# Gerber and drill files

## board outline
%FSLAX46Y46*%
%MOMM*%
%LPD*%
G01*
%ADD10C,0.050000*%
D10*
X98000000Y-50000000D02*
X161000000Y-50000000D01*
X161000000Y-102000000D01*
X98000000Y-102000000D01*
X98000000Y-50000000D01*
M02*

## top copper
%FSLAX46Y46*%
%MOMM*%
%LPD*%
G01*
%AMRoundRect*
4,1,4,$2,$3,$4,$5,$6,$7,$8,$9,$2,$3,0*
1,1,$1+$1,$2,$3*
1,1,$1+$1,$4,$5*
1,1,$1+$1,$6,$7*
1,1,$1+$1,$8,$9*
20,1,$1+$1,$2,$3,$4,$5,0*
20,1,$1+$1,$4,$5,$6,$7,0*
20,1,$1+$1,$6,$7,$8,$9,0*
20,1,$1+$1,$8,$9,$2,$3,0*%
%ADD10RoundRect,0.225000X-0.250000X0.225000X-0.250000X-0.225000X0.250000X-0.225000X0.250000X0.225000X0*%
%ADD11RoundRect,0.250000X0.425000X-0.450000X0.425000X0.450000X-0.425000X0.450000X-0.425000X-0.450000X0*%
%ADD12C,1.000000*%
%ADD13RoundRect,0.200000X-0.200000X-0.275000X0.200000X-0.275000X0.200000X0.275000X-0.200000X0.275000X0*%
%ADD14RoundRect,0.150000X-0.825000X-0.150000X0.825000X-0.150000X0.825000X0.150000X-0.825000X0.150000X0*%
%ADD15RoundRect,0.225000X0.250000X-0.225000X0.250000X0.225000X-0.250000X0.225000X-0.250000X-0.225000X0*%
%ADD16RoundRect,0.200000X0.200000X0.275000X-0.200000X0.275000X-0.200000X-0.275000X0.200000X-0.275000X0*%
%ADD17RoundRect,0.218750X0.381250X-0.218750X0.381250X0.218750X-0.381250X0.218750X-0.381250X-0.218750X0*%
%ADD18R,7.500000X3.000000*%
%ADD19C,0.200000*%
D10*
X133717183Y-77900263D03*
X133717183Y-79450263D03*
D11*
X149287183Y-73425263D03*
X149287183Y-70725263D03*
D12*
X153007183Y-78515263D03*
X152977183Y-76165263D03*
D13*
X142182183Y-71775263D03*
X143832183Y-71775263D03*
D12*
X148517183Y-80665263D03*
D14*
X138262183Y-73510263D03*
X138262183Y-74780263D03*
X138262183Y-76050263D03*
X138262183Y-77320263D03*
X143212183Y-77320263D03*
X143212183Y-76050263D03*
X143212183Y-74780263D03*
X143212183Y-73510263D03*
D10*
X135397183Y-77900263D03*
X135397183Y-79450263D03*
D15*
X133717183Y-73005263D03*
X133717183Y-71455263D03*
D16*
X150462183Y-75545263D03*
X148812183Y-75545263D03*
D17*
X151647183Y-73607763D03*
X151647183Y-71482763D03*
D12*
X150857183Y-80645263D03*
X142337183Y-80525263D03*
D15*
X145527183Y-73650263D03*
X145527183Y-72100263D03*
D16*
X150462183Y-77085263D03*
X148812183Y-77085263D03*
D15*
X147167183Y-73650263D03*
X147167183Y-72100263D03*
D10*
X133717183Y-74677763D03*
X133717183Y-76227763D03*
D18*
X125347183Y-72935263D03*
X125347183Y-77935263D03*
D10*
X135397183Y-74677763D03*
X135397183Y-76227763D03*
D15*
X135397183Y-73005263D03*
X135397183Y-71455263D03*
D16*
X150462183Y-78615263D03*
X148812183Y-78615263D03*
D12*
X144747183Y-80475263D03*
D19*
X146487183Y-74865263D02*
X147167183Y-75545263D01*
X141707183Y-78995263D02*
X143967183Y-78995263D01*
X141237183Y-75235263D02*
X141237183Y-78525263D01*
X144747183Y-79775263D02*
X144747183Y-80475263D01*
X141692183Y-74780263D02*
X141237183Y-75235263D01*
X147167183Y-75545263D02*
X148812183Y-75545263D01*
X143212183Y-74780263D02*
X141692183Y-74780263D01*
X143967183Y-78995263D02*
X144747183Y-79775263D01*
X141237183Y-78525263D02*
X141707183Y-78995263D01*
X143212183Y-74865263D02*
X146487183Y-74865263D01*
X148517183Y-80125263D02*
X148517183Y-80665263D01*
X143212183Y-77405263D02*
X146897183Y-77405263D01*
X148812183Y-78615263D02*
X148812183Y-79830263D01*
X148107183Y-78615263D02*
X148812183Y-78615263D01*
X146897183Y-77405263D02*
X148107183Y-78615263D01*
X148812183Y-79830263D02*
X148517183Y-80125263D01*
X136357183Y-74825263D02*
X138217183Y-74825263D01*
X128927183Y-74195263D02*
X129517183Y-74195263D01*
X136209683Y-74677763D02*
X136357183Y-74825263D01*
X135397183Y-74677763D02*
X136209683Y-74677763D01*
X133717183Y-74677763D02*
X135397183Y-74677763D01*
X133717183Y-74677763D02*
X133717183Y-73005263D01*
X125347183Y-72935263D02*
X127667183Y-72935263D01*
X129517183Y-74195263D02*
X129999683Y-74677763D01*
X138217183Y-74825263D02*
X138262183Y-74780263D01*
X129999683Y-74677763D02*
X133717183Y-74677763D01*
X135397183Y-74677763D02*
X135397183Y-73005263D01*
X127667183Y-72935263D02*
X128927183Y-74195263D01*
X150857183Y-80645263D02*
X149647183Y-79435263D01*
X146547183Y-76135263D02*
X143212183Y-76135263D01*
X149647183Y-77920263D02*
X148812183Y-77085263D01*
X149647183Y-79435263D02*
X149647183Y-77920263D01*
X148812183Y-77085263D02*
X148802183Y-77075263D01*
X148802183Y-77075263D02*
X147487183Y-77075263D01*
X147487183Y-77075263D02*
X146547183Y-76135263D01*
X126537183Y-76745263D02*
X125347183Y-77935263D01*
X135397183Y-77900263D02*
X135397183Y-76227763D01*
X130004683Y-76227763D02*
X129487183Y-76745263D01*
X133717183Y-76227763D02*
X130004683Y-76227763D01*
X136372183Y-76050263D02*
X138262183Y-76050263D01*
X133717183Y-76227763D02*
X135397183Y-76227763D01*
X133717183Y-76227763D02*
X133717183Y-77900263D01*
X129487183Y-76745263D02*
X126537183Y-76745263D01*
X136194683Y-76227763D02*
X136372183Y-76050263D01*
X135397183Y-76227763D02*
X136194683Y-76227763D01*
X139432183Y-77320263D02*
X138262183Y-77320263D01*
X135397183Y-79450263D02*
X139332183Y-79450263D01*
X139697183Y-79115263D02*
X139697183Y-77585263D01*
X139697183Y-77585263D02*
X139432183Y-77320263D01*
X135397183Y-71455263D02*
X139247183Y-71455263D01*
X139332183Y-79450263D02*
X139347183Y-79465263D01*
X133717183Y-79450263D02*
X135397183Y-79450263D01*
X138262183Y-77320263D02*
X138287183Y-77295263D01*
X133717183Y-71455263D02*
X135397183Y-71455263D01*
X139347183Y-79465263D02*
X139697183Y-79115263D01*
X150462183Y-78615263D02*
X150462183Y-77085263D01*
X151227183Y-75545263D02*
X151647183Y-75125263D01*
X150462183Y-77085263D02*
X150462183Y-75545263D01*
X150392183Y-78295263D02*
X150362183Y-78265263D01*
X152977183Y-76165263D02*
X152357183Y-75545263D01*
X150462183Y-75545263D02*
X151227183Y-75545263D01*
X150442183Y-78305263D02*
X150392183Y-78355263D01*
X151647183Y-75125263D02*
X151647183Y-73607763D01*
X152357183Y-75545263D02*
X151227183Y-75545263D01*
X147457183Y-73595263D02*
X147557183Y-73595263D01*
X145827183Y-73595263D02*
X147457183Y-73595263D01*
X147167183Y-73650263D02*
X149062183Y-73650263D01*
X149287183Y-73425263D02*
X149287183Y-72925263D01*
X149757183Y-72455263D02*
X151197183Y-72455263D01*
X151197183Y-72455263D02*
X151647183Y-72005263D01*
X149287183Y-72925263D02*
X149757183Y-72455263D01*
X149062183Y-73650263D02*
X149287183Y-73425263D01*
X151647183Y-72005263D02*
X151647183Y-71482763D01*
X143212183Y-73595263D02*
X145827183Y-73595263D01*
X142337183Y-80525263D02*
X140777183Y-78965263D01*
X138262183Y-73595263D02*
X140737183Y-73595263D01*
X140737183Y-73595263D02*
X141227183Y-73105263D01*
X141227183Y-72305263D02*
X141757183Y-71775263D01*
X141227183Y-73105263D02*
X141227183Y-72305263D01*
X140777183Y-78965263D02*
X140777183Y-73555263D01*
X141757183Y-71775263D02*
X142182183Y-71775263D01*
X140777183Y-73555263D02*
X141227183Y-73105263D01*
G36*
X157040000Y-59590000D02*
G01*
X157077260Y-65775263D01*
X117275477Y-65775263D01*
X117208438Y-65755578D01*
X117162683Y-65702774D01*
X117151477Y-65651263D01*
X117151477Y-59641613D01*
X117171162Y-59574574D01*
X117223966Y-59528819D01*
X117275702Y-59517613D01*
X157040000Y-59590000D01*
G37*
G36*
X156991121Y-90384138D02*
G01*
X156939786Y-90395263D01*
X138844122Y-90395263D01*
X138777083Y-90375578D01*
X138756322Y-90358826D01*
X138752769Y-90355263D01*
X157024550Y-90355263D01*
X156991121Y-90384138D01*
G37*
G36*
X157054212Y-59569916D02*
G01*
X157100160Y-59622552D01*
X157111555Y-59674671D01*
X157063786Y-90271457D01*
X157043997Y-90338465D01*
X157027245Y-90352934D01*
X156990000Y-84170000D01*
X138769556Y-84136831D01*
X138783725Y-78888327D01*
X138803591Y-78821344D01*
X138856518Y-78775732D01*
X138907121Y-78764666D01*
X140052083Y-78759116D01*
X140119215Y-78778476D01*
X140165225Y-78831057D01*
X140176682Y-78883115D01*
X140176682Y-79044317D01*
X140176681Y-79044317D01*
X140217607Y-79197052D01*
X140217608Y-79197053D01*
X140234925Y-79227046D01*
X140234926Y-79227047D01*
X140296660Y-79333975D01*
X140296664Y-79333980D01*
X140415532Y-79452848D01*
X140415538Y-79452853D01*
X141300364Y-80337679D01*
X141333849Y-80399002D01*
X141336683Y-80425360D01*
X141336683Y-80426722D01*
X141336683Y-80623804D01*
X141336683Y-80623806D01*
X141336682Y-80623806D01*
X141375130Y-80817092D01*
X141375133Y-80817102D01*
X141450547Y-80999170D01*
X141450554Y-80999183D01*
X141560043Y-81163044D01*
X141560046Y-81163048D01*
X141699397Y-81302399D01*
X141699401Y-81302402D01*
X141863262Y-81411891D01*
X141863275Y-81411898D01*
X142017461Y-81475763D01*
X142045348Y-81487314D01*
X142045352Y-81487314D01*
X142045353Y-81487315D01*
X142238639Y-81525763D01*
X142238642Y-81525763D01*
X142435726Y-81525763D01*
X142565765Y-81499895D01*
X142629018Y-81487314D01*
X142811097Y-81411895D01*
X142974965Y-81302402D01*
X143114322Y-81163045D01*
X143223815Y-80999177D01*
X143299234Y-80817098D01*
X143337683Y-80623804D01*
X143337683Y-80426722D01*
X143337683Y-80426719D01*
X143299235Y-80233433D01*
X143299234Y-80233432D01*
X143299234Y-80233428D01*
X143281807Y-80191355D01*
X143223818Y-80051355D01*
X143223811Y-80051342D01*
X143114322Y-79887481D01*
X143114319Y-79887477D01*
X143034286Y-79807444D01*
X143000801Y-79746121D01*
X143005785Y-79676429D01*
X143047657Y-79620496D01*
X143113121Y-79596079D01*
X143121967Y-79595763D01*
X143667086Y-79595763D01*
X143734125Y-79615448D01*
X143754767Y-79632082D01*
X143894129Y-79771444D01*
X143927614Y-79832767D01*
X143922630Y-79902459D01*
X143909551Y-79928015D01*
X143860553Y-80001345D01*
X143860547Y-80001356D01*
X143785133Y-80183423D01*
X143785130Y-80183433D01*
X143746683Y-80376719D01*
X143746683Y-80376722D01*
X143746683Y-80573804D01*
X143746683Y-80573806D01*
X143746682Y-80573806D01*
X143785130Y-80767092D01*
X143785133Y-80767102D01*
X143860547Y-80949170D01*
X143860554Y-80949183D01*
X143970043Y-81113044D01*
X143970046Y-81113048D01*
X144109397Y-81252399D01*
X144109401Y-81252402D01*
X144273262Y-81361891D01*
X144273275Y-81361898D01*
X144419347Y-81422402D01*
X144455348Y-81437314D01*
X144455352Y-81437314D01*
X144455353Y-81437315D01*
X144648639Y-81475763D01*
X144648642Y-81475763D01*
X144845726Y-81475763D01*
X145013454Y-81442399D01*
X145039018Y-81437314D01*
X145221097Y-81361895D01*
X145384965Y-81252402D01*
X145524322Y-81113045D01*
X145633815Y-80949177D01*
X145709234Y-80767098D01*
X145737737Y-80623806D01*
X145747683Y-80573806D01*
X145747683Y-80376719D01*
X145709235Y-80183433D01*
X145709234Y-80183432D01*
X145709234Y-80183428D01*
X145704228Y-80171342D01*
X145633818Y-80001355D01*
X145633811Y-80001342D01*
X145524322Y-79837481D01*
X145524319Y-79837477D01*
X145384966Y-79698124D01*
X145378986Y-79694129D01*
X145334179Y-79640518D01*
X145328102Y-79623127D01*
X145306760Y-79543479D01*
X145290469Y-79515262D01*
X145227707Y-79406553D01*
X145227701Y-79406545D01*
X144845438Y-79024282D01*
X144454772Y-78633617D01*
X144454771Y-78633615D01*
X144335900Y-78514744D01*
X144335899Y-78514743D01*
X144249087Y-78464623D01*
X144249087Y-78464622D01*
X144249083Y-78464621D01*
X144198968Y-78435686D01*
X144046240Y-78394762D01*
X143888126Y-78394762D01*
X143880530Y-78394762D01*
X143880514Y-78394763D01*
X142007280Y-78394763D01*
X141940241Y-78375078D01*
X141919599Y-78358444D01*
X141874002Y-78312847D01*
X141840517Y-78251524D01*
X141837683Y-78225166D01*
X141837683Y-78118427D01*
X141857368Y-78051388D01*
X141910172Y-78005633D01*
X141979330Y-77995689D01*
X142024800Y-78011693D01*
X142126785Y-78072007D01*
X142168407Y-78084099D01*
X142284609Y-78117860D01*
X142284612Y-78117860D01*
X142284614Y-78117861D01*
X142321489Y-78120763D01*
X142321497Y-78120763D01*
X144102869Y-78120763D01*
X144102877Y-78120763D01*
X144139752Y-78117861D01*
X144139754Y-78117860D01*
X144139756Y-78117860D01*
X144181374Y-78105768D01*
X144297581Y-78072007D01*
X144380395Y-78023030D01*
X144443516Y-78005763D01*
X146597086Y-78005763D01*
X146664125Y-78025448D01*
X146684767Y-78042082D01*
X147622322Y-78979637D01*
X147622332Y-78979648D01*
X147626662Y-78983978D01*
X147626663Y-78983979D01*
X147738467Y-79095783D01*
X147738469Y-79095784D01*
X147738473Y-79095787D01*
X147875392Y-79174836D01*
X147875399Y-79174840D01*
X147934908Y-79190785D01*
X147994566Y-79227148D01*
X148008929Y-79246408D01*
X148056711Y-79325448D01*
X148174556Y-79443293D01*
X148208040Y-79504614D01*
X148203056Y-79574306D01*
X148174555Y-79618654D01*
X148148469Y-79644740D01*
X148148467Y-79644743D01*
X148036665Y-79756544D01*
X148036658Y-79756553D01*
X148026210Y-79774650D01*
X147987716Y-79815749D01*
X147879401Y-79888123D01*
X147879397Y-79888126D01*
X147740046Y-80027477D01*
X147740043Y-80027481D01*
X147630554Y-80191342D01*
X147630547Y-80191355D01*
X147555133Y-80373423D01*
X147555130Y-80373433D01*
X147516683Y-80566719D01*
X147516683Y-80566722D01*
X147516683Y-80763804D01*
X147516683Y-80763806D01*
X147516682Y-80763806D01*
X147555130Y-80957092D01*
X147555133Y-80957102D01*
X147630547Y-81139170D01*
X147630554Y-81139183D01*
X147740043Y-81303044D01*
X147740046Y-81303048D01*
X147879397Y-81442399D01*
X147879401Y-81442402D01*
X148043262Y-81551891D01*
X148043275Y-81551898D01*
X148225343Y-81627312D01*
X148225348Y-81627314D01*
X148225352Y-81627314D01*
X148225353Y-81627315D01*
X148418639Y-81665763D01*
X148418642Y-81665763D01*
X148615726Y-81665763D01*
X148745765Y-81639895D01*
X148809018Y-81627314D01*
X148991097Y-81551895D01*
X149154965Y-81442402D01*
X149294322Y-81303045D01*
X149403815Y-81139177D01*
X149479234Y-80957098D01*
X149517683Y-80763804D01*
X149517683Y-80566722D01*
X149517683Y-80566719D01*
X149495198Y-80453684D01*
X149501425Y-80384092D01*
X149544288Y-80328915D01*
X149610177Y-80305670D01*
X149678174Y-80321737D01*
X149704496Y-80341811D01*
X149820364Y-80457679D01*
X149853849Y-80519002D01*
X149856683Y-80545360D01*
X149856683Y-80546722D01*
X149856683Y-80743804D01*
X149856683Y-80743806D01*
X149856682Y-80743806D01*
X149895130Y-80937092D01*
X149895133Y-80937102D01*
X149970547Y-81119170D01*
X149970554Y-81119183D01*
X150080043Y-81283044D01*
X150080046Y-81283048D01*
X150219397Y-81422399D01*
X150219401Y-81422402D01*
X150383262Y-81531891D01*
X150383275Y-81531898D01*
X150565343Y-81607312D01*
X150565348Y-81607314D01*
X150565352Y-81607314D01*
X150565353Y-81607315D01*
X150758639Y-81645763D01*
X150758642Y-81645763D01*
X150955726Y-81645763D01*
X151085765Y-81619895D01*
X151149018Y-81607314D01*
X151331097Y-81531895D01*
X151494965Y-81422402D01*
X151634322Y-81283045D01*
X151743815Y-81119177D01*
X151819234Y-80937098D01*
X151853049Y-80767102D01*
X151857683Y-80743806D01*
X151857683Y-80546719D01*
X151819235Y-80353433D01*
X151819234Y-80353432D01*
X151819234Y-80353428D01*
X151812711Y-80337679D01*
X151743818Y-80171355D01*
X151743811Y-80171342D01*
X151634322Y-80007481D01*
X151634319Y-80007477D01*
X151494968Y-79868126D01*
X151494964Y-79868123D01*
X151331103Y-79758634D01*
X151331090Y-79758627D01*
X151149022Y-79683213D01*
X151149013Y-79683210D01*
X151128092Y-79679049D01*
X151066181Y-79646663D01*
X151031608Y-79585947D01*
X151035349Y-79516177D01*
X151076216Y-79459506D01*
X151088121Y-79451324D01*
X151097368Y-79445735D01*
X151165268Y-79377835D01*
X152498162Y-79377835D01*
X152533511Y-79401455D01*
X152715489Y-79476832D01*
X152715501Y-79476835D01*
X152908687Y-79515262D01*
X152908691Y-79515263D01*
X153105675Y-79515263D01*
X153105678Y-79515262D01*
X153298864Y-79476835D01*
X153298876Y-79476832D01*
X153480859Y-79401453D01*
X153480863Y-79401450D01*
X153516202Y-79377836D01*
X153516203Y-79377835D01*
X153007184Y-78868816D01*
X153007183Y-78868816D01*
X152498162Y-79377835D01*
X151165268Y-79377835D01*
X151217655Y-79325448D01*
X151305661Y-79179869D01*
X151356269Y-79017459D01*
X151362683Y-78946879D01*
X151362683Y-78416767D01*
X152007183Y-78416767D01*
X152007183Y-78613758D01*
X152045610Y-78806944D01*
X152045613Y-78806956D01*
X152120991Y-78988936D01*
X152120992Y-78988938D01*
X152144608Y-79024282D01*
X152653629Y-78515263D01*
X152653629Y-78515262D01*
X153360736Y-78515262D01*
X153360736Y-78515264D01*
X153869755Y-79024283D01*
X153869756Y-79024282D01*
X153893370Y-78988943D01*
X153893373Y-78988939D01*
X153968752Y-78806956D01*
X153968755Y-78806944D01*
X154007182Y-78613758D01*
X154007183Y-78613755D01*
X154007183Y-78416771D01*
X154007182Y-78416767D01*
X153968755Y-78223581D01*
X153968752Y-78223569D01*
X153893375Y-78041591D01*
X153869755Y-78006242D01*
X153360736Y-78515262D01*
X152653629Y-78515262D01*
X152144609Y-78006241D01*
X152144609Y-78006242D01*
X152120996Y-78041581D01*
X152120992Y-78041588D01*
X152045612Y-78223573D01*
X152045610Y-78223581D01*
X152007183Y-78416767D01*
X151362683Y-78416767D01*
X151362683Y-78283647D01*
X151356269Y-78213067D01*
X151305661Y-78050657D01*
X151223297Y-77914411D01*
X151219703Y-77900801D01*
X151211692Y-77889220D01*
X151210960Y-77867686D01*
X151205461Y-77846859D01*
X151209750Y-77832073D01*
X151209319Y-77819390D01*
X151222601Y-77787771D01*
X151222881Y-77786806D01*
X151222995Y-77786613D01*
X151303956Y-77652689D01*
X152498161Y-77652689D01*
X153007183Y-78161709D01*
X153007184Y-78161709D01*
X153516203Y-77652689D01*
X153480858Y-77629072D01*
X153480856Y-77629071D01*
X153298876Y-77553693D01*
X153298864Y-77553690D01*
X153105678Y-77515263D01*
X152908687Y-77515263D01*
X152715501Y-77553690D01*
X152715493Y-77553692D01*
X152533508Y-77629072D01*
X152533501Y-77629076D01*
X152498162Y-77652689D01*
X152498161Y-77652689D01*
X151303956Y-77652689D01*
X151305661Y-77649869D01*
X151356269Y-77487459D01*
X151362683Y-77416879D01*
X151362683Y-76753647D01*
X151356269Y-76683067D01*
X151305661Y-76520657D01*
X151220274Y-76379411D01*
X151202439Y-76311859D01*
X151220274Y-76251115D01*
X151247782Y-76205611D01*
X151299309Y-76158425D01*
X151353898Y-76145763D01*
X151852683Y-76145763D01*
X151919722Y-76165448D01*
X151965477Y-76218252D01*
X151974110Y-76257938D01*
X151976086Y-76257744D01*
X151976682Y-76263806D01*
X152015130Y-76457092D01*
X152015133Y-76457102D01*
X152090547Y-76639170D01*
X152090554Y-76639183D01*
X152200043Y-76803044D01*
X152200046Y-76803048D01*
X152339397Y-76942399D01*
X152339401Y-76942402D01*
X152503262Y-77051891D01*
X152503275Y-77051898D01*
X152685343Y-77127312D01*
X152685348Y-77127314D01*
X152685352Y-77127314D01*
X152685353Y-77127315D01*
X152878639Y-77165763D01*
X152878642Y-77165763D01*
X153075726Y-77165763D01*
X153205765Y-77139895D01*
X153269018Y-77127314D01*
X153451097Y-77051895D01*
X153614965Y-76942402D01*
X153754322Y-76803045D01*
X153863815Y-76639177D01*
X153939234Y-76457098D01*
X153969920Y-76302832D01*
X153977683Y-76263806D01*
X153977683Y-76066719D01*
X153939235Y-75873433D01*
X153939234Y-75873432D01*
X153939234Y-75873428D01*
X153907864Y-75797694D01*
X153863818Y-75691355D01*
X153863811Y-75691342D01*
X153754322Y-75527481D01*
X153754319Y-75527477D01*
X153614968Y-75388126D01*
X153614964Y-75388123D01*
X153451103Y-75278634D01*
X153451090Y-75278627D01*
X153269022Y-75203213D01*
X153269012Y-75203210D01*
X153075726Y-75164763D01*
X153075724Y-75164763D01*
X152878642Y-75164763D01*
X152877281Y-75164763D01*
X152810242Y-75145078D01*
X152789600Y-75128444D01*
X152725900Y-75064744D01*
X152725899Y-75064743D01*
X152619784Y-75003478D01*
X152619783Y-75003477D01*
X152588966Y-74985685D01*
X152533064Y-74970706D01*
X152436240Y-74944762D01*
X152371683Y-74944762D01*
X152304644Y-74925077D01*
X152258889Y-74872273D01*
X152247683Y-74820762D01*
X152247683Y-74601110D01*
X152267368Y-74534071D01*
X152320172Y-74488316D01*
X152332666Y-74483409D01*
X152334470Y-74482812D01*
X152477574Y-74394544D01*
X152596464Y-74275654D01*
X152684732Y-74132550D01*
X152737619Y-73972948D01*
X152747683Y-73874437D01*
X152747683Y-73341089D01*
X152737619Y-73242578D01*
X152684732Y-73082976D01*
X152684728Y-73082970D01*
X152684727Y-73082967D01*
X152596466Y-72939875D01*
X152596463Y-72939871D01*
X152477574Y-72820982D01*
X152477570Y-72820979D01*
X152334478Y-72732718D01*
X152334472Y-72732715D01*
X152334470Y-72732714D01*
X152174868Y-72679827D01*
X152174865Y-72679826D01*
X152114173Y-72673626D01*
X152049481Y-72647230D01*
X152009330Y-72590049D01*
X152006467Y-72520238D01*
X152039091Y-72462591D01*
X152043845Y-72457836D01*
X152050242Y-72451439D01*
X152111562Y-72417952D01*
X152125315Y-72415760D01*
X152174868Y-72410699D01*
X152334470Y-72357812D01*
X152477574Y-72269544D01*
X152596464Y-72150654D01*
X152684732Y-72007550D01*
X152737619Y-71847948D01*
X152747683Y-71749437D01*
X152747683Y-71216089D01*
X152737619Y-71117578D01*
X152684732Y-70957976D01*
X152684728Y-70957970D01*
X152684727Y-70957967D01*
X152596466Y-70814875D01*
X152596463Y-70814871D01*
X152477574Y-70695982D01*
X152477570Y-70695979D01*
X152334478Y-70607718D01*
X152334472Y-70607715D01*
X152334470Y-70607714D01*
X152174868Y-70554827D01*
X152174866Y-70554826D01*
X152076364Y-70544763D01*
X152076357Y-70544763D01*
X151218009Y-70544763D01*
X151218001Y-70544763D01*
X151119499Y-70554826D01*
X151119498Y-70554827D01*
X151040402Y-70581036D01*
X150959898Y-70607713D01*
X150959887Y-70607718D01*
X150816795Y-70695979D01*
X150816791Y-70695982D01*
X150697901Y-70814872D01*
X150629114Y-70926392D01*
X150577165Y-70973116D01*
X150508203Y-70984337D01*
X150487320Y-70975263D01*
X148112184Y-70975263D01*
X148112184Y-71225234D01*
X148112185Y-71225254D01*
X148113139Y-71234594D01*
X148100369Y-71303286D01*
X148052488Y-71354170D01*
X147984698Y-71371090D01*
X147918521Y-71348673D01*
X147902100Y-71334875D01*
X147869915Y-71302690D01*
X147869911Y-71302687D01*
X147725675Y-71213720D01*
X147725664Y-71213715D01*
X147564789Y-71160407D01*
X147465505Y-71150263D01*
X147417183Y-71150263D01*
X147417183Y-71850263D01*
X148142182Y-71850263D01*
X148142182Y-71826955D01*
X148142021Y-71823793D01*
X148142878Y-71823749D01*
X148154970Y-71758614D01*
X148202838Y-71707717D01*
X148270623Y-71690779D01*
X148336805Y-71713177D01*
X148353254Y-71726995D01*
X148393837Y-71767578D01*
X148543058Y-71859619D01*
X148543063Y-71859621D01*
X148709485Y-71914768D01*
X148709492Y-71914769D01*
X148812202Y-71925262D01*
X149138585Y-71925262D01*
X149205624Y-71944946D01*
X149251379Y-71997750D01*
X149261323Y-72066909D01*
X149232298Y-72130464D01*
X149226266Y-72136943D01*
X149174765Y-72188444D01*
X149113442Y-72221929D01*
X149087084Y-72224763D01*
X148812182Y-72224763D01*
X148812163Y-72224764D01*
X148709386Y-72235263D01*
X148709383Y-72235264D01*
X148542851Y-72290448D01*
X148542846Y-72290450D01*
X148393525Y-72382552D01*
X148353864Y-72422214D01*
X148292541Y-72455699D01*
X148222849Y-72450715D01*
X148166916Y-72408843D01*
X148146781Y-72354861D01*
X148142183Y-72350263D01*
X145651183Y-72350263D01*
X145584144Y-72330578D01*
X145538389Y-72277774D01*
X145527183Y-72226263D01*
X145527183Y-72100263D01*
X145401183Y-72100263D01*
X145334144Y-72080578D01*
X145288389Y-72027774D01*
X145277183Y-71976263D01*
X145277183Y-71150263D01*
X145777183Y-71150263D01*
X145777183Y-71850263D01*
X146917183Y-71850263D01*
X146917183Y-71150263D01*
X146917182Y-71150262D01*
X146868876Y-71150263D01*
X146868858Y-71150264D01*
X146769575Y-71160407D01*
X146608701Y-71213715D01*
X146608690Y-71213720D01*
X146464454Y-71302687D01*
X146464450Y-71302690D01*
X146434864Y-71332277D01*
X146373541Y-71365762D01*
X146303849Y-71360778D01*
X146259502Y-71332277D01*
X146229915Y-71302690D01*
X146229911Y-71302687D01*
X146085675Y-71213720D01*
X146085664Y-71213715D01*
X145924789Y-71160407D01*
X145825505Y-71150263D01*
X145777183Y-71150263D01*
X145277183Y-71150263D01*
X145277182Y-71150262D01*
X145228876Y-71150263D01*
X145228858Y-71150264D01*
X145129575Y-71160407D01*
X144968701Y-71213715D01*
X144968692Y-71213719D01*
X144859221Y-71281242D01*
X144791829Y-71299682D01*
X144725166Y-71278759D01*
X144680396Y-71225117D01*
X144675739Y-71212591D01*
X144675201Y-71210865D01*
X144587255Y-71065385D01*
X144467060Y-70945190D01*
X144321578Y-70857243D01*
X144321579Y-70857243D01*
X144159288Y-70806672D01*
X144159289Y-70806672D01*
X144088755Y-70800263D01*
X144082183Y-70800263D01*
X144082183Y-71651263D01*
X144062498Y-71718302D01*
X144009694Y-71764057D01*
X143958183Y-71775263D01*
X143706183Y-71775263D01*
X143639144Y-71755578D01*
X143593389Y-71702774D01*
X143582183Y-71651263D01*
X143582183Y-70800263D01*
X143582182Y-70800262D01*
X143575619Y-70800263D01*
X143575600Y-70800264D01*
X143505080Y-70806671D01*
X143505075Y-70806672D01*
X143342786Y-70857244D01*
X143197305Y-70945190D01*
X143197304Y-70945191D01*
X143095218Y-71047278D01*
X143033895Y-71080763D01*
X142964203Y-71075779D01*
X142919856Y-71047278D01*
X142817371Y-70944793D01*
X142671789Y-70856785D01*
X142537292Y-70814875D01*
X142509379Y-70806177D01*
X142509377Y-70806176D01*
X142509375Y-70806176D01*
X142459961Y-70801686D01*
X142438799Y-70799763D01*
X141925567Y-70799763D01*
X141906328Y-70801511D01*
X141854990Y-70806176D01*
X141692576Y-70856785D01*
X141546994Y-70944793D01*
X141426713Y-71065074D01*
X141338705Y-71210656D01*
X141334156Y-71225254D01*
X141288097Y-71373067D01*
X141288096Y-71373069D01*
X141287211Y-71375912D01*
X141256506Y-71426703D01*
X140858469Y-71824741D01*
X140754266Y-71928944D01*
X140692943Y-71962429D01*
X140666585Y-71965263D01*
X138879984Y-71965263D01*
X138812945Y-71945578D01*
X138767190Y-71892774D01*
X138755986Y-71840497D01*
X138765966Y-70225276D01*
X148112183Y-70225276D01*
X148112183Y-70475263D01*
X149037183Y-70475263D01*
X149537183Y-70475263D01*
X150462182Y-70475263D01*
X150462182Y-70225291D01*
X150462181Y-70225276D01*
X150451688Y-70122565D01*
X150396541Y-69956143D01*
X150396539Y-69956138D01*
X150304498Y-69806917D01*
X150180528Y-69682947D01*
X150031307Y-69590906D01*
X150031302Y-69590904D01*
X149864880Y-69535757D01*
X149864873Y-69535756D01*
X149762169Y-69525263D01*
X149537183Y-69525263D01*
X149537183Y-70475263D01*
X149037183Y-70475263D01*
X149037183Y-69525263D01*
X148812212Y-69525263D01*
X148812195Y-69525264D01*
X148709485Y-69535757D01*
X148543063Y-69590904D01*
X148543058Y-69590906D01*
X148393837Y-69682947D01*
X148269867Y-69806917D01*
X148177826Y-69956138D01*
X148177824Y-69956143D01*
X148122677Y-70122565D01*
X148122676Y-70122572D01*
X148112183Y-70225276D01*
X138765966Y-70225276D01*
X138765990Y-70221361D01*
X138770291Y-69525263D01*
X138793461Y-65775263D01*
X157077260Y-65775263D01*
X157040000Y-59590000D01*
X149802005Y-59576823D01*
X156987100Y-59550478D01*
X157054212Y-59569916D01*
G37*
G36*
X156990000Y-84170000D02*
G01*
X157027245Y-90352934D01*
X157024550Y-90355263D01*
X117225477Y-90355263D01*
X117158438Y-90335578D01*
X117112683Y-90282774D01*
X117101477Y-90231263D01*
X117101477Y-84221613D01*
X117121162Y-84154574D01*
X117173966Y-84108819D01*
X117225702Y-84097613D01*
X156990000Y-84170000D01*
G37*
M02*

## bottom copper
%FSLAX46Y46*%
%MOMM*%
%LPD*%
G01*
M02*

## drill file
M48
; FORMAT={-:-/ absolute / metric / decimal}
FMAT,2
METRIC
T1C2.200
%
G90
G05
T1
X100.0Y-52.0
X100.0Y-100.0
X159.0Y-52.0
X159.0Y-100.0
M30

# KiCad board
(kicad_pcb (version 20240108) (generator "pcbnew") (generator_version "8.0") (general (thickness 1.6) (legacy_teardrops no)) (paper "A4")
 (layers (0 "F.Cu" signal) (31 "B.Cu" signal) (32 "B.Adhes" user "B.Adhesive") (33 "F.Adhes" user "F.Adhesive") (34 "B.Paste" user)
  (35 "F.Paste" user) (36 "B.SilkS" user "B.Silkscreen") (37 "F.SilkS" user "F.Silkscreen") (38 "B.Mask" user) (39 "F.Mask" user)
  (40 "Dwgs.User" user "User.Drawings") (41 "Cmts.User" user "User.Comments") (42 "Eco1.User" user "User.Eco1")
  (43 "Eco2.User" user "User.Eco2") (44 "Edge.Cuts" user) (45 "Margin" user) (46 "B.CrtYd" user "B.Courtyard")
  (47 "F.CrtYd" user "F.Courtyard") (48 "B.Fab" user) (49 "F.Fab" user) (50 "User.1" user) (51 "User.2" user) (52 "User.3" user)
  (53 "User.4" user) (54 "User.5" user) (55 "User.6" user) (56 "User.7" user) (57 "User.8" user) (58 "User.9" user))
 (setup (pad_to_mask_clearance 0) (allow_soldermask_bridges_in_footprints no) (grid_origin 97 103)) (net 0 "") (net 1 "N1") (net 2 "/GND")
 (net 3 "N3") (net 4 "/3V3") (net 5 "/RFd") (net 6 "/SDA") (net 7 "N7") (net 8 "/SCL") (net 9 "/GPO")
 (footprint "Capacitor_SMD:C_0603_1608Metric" (layer "F.Cu") (at 133.717183 78.675263 -90)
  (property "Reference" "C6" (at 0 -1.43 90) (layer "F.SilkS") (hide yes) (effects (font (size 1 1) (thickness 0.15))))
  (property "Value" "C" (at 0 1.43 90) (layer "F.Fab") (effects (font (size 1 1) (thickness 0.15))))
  (pad "1" smd roundrect (at -0.775 0 270) (size 0.9 0.95) (layers "F.Cu" "F.Paste" "F.Mask") (roundrect_rratio 0.25) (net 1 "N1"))
  (pad "2" smd roundrect (at 0.775 0 270) (size 0.9 0.95) (layers "F.Cu" "F.Paste" "F.Mask") (roundrect_rratio 0.25) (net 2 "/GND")))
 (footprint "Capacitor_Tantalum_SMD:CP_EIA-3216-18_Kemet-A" (layer "F.Cu") (at 149.287183 72.075263 90)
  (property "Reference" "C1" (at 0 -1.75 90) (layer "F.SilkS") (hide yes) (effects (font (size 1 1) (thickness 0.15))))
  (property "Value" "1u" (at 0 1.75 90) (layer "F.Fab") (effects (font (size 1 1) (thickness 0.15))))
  (pad "1" smd roundrect (at -1.35 0 90) (size 1.4 1.35) (layers "F.Cu" "F.Paste" "F.Mask") (roundrect_rratio 0.185185) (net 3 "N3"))
  (pad "2" smd roundrect (at 1.35 0 90) (size 1.4 1.35) (layers "F.Cu" "F.Paste" "F.Mask") (roundrect_rratio 0.185185) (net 2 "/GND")))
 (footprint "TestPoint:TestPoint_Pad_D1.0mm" (layer "F.Cu") (at 153.007183 78.515263)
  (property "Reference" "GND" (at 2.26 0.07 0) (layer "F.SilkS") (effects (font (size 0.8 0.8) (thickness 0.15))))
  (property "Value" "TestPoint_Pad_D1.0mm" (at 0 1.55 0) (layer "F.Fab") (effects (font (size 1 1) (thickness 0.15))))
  (pad "1" smd circle (at 0 0) (size 1 1) (layers "F.Cu" "F.Mask") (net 2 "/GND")))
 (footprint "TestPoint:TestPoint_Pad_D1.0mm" (layer "F.Cu") (at 152.977183 76.165263)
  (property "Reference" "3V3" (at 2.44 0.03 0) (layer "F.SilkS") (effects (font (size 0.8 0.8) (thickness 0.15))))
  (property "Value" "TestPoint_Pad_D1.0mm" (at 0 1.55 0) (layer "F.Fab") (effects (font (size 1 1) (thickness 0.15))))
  (pad "2" smd circle (at 0 0) (size 1 1) (layers "F.Cu" "F.Mask") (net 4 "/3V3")))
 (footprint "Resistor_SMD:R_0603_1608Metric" (layer "F.Cu") (at 143.007183 71.775263)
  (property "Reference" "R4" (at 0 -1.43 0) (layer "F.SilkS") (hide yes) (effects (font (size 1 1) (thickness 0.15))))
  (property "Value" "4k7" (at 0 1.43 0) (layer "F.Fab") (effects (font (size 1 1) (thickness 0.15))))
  (pad "1" smd roundrect (at -0.825 0) (size 0.8 0.95) (layers "F.Cu" "F.Paste" "F.Mask") (roundrect_rratio 0.25) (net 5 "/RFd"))
  (pad "2" smd roundrect (at 0.825 0) (size 0.8 0.95) (layers "F.Cu" "F.Paste" "F.Mask") (roundrect_rratio 0.25) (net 2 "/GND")))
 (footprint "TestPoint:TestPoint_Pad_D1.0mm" (layer "F.Cu") (at 148.517183 80.665263)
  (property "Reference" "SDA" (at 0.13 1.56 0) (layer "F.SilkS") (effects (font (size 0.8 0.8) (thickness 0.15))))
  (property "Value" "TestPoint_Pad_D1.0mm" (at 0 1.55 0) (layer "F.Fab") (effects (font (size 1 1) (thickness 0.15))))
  (pad "3" smd circle (at 0 0) (size 1 1) (layers "F.Cu" "F.Mask") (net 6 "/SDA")))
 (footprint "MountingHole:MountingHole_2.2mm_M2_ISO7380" (layer "F.Cu") (at 100 52)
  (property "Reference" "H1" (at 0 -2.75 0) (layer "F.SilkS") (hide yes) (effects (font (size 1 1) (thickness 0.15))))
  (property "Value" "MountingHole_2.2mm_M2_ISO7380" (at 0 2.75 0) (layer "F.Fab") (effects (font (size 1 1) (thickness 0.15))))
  (pad "" np_thru_hole circle (at 0 0) (size 2.2 2.2) (drill 2.2) (layers "*.Cu" "*.Mask")))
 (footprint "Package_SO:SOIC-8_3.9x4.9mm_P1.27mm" (layer "F.Cu") (at 140.737183 75.415263)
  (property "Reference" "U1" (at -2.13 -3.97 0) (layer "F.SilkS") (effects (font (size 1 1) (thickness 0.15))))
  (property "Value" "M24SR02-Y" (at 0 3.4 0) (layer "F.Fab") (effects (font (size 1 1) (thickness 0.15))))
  (pad "1" smd roundrect (at -2.475 -1.905) (size 1.95 0.6) (layers "F.Cu" "F.Paste" "F.Mask") (roundrect_rratio 0.25) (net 5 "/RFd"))
  (pad "2" smd roundrect (at -2.475 -0.635) (size 1.95 0.6) (layers "F.Cu" "F.Paste" "F.Mask") (roundrect_rratio 0.25) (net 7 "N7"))
  (pad "3" smd roundrect (at -2.475 0.635) (size 1.95 0.6) (layers "F.Cu" "F.Paste" "F.Mask") (roundrect_rratio 0.25) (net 1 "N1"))
  (pad "4" smd roundrect (at -2.475 1.905) (size 1.95 0.6) (layers "F.Cu" "F.Paste" "F.Mask") (roundrect_rratio 0.25) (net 2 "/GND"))
  (pad "5" smd roundrect (at 2.475 1.905) (size 1.95 0.6) (layers "F.Cu" "F.Paste" "F.Mask") (roundrect_rratio 0.25) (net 6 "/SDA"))
  (pad "6" smd roundrect (at 2.475 0.635) (size 1.95 0.6) (layers "F.Cu" "F.Paste" "F.Mask") (roundrect_rratio 0.25) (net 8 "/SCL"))
  (pad "7" smd roundrect (at 2.475 -0.635) (size 1.95 0.6) (layers "F.Cu" "F.Paste" "F.Mask") (roundrect_rratio 0.25) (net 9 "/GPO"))
  (pad "8" smd roundrect (at 2.475 -1.905) (size 1.95 0.6) (layers "F.Cu" "F.Paste" "F.Mask") (roundrect_rratio 0.25) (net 3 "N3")))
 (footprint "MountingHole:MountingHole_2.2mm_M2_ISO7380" (layer "F.Cu") (at 159 100)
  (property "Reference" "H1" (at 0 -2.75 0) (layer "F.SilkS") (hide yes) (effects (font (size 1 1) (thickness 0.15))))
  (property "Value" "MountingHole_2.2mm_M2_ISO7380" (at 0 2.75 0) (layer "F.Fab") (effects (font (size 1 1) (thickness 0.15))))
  (pad "" np_thru_hole circle (at 0 0) (size 2.2 2.2) (drill 2.2) (layers "*.Cu" "*.Mask")))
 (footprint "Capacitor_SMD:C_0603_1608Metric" (layer "F.Cu") (at 135.397183 78.675263 -90)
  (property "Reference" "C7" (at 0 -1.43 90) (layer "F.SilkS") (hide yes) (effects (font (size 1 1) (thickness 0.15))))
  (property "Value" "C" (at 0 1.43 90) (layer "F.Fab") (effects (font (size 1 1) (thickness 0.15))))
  (pad "1" smd roundrect (at -0.775 0 270) (size 0.9 0.95) (layers "F.Cu" "F.Paste" "F.Mask") (roundrect_rratio 0.25) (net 1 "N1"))
  (pad "2" smd roundrect (at 0.775 0 270) (size 0.9 0.95) (layers "F.Cu" "F.Paste" "F.Mask") (roundrect_rratio 0.25) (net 2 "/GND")))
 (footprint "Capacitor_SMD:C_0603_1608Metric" (layer "F.Cu") (at 133.717183 72.230263 90)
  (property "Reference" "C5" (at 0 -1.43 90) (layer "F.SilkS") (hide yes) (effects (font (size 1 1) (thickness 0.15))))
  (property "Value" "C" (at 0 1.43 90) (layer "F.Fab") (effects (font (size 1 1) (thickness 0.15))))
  (pad "1" smd roundrect (at -0.775 0 90) (size 0.9 0.95) (layers "F.Cu" "F.Paste" "F.Mask") (roundrect_rratio 0.25) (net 7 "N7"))
  (pad "2" smd roundrect (at 0.775 0 90) (size 0.9 0.95) (layers "F.Cu" "F.Paste" "F.Mask") (roundrect_rratio 0.25) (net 2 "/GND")))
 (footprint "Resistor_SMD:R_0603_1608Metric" (layer "F.Cu") (at 149.637183 75.545263 180)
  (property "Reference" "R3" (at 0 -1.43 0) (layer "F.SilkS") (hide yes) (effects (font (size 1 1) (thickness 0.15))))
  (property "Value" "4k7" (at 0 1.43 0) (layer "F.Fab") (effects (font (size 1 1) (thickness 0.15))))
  (pad "1" smd roundrect (at -0.825 0 180) (size 0.8 0.95) (layers "F.Cu" "F.Paste" "F.Mask") (roundrect_rratio 0.25) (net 4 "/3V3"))
  (pad "2" smd roundrect (at 0.825 0 180) (size 0.8 0.95) (layers "F.Cu" "F.Paste" "F.Mask") (roundrect_rratio 0.25) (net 9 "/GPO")))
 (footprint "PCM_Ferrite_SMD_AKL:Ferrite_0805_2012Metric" (layer "F.Cu") (at 151.647183 72.545263 90)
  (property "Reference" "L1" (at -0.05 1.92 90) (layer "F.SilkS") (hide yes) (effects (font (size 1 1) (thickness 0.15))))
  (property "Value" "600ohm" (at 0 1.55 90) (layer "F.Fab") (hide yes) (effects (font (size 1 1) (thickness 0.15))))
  (pad "1" smd roundrect (at -1.0625 0 90) (size 0.875 1.2) (layers "F.Cu" "F.Paste" "F.Mask") (roundrect_rratio 0.25) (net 4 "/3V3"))
  (pad "2" smd roundrect (at 1.0625 0 90) (size 0.875 1.2) (layers "F.Cu" "F.Paste" "F.Mask") (roundrect_rratio 0.25) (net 3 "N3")))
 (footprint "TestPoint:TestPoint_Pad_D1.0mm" (layer "F.Cu") (at 150.857183 80.645263)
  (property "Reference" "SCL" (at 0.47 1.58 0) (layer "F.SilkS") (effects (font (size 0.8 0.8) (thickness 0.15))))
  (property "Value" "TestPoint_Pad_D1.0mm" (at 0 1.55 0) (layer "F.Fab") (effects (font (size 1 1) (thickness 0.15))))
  (pad "4" smd circle (at 0 0) (size 1 1) (layers "F.Cu" "F.Mask") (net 8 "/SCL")))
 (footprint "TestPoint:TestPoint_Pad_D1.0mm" (layer "F.Cu") (at 142.337183 80.525263)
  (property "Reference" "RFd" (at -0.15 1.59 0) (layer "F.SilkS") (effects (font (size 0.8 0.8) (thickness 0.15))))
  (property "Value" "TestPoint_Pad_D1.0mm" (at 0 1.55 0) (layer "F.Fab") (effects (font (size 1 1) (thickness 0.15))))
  (pad "6" smd circle (at 0 0) (size 1 1) (layers "F.Cu" "F.Mask") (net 5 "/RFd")))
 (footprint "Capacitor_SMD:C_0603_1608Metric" (layer "F.Cu") (at 145.527183 72.875263 90)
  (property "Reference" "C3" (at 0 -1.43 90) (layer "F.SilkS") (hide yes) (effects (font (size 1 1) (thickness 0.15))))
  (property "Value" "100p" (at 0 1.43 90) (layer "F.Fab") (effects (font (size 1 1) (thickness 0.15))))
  (pad "1" smd roundrect (at -0.775 0 90) (size 0.9 0.95) (layers "F.Cu" "F.Paste" "F.Mask") (roundrect_rratio 0.25) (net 3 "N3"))
  (pad "2" smd roundrect (at 0.775 0 90) (size 0.9 0.95) (layers "F.Cu" "F.Paste" "F.Mask") (roundrect_rratio 0.25) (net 2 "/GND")))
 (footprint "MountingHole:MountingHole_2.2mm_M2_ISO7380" (layer "F.Cu") (at 100 100)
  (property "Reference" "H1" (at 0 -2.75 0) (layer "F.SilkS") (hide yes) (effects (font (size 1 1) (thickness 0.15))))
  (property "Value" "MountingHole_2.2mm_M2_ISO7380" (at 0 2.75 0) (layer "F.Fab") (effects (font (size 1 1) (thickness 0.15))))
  (pad "" np_thru_hole circle (at 0 0) (size 2.2 2.2) (drill 2.2) (layers "*.Cu" "*.Mask")))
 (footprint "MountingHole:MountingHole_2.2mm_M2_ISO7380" (layer "F.Cu") (at 159 52)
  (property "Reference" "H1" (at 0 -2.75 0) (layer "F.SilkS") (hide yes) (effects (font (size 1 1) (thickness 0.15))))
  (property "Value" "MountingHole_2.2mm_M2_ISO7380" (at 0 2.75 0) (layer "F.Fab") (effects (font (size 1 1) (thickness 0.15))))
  (pad "" np_thru_hole circle (at 0 0) (size 2.2 2.2) (drill 2.2) (layers "*.Cu" "*.Mask")))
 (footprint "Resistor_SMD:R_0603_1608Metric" (layer "F.Cu") (at 149.637183 77.085263 180)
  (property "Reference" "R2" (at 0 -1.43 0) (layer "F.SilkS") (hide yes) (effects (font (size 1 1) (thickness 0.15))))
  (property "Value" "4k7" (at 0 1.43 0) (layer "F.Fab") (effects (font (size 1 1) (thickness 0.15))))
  (pad "1" smd roundrect (at -0.825 0 180) (size 0.8 0.95) (layers "F.Cu" "F.Paste" "F.Mask") (roundrect_rratio 0.25) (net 4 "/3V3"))
  (pad "2" smd roundrect (at 0.825 0 180) (size 0.8 0.95) (layers "F.Cu" "F.Paste" "F.Mask") (roundrect_rratio 0.25) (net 8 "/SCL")))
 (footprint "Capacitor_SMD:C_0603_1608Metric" (layer "F.Cu") (at 147.167183 72.875263 90)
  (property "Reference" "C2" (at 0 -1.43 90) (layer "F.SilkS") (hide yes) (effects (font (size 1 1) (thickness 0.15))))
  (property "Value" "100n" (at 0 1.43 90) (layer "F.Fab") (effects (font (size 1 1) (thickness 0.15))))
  (pad "1" smd roundrect (at -0.775 0 90) (size 0.9 0.95) (layers "F.Cu" "F.Paste" "F.Mask") (roundrect_rratio 0.25) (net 3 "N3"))
  (pad "2" smd roundrect (at 0.775 0 90) (size 0.9 0.95) (layers "F.Cu" "F.Paste" "F.Mask") (roundrect_rratio 0.25) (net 2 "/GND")))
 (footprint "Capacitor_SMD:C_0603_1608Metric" (layer "F.Cu") (at 133.717183 75.452763 -90)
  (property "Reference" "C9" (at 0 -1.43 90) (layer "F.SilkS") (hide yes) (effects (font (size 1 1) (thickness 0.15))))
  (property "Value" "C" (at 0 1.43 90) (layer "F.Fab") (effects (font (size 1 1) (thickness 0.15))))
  (pad "1" smd roundrect (at -0.775 0 270) (size 0.9 0.95) (layers "F.Cu" "F.Paste" "F.Mask") (roundrect_rratio 0.25) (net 7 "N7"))
  (pad "2" smd roundrect (at 0.775 0 270) (size 0.9 0.95) (layers "F.Cu" "F.Paste" "F.Mask") (roundrect_rratio 0.25) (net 1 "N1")))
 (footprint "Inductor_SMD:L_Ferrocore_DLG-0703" (layer "F.Cu") (at 125.347183 75.435263 -90)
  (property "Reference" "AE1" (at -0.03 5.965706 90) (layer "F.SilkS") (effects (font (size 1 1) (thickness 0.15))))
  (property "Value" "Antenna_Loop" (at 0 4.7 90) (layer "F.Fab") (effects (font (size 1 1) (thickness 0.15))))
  (pad "1" smd rect (at -2.5 0 270) (size 3 7.5) (layers "F.Cu" "F.Paste" "F.Mask") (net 7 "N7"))
  (pad "2" smd rect (at 2.5 0 270) (size 3 7.5) (layers "F.Cu" "F.Paste" "F.Mask") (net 1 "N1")))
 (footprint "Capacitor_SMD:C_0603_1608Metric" (layer "F.Cu") (at 135.397183 75.452763 -90)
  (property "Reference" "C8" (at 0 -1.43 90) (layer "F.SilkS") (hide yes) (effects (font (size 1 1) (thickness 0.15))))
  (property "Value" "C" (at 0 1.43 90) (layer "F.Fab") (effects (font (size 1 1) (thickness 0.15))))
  (pad "1" smd roundrect (at -0.775 0 270) (size 0.9 0.95) (layers "F.Cu" "F.Paste" "F.Mask") (roundrect_rratio 0.25) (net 7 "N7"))
  (pad "2" smd roundrect (at 0.775 0 270) (size 0.9 0.95) (layers "F.Cu" "F.Paste" "F.Mask") (roundrect_rratio 0.25) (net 1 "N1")))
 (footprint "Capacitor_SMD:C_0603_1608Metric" (layer "F.Cu") (at 135.397183 72.230263 90)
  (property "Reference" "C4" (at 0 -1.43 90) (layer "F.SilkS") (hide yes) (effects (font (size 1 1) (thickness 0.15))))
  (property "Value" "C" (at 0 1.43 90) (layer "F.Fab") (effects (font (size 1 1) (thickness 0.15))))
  (pad "1" smd roundrect (at -0.775 0 90) (size 0.9 0.95) (layers "F.Cu" "F.Paste" "F.Mask") (roundrect_rratio 0.25) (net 7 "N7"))
  (pad "2" smd roundrect (at 0.775 0 90) (size 0.9 0.95) (layers "F.Cu" "F.Paste" "F.Mask") (roundrect_rratio 0.25) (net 2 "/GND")))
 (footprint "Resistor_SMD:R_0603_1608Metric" (layer "F.Cu") (at 149.637183 78.615263 180)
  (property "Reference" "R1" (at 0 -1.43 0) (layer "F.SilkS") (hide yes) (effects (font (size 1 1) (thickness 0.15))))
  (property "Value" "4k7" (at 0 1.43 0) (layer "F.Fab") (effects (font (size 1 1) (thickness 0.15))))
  (pad "1" smd roundrect (at -0.825 0 180) (size 0.8 0.95) (layers "F.Cu" "F.Paste" "F.Mask") (roundrect_rratio 0.25) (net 4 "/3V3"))
  (pad "2" smd roundrect (at 0.825 0 180) (size 0.8 0.95) (layers "F.Cu" "F.Paste" "F.Mask") (roundrect_rratio 0.25) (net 6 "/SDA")))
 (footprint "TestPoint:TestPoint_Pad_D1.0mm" (layer "F.Cu") (at 144.747183 80.475263)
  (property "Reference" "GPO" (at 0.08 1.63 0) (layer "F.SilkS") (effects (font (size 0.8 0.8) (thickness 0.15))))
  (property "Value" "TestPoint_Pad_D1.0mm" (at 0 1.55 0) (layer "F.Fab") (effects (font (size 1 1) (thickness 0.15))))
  (pad "5" smd circle (at 0 0) (size 1 1) (layers "F.Cu" "F.Mask") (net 9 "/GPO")))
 (gr_rect (start 98 50) (end 161 102) (stroke (width 0.05) (type default)) (fill none) (layer "Edge.Cuts"))
 (segment (start 146.487183 74.865263) (end 147.167183 75.545263) (width 0.2) (layer "F.Cu") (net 9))
 (segment (start 141.707183 78.995263) (end 143.967183 78.995263) (width 0.2) (layer "F.Cu") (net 9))
 (segment (start 141.237183 75.235263) (end 141.237183 78.525263) (width 0.2) (layer "F.Cu") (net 9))
 (segment (start 144.747183 79.775263) (end 144.747183 80.475263) (width 0.2) (layer "F.Cu") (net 9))
 (segment (start 141.692183 74.780263) (end 141.237183 75.235263) (width 0.2) (layer "F.Cu") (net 9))
 (segment (start 147.167183 75.545263) (end 148.812183 75.545263) (width 0.2) (layer "F.Cu") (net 9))
 (segment (start 143.212183 74.780263) (end 141.692183 74.780263) (width 0.2) (layer "F.Cu") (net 9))
 (segment (start 143.967183 78.995263) (end 144.747183 79.775263) (width 0.2) (layer "F.Cu") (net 9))
 (segment (start 141.237183 78.525263) (end 141.707183 78.995263) (width 0.2) (layer "F.Cu") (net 9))
 (segment (start 143.212183 74.865263) (end 146.487183 74.865263) (width 0.2) (layer "F.Cu") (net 9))
 (segment (start 148.517183 80.125263) (end 148.517183 80.665263) (width 0.2) (layer "F.Cu") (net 6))
 (segment (start 143.212183 77.405263) (end 146.897183 77.405263) (width 0.2) (layer "F.Cu") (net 6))
 (segment (start 148.812183 78.615263) (end 148.812183 79.830263) (width 0.2) (layer "F.Cu") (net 6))
 (segment (start 148.107183 78.615263) (end 148.812183 78.615263) (width 0.2) (layer "F.Cu") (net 6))
 (segment (start 146.897183 77.405263) (end 148.107183 78.615263) (width 0.2) (layer "F.Cu") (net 6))
 (segment (start 148.812183 79.830263) (end 148.517183 80.125263) (width 0.2) (layer "F.Cu") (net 6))
 (segment (start 136.357183 74.825263) (end 138.217183 74.825263) (width 0.2) (layer "F.Cu") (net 7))
 (segment (start 128.927183 74.195263) (end 129.517183 74.195263) (width 0.2) (layer "F.Cu") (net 7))
 (segment (start 136.209683 74.677763) (end 136.357183 74.825263) (width 0.2) (layer "F.Cu") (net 7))
 (segment (start 135.397183 74.677763) (end 136.209683 74.677763) (width 0.2) (layer "F.Cu") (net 7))
 (segment (start 133.717183 74.677763) (end 135.397183 74.677763) (width 0.2) (layer "F.Cu") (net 7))
 (segment (start 133.717183 74.677763) (end 133.717183 73.005263) (width 0.2) (layer "F.Cu") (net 7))
 (segment (start 125.347183 72.935263) (end 127.667183 72.935263) (width 0.2) (layer "F.Cu") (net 7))
 (segment (start 129.517183 74.195263) (end 129.999683 74.677763) (width 0.2) (layer "F.Cu") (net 7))
 (segment (start 138.217183 74.825263) (end 138.262183 74.780263) (width 0.2) (layer "F.Cu") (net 7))
 (segment (start 129.999683 74.677763) (end 133.717183 74.677763) (width 0.2) (layer "F.Cu") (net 7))
 (segment (start 135.397183 74.677763) (end 135.397183 73.005263) (width 0.2) (layer "F.Cu") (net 7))
 (segment (start 127.667183 72.935263) (end 128.927183 74.195263) (width 0.2) (layer "F.Cu") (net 7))
 (segment (start 150.857183 80.645263) (end 149.647183 79.435263) (width 0.2) (layer "F.Cu") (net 8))
 (segment (start 146.547183 76.135263) (end 143.212183 76.135263) (width 0.2) (layer "F.Cu") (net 8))
 (segment (start 149.647183 77.920263) (end 148.812183 77.085263) (width 0.2) (layer "F.Cu") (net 8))
 (segment (start 149.647183 79.435263) (end 149.647183 77.920263) (width 0.2) (layer "F.Cu") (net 8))
 (segment (start 148.812183 77.085263) (end 148.802183 77.075263) (width 0.2) (layer "F.Cu") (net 8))
 (segment (start 148.802183 77.075263) (end 147.487183 77.075263) (width 0.2) (layer "F.Cu") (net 8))
 (segment (start 147.487183 77.075263) (end 146.547183 76.135263) (width 0.2) (layer "F.Cu") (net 8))
 (segment (start 126.537183 76.745263) (end 125.347183 77.935263) (width 0.2) (layer "F.Cu") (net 1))
 (segment (start 135.397183 77.900263) (end 135.397183 76.227763) (width 0.2) (layer "F.Cu") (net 1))
 (segment (start 130.004683 76.227763) (end 129.487183 76.745263) (width 0.2) (layer "F.Cu") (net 1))
 (segment (start 133.717183 76.227763) (end 130.004683 76.227763) (width 0.2) (layer "F.Cu") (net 1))
 (segment (start 136.372183 76.050263) (end 138.262183 76.050263) (width 0.2) (layer "F.Cu") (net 1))
 (segment (start 133.717183 76.227763) (end 135.397183 76.227763) (width 0.2) (layer "F.Cu") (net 1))
 (segment (start 133.717183 76.227763) (end 133.717183 77.900263) (width 0.2) (layer "F.Cu") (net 1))
 (segment (start 129.487183 76.745263) (end 126.537183 76.745263) (width 0.2) (layer "F.Cu") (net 1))
 (segment (start 136.194683 76.227763) (end 136.372183 76.050263) (width 0.2) (layer "F.Cu") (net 1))
 (segment (start 135.397183 76.227763) (end 136.194683 76.227763) (width 0.2) (layer "F.Cu") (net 1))
 (segment (start 139.432183 77.320263) (end 138.262183 77.320263) (width 0.2) (layer "F.Cu") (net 2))
 (segment (start 135.397183 79.450263) (end 139.332183 79.450263) (width 0.2) (layer "F.Cu") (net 2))
 (segment (start 139.697183 79.115263) (end 139.697183 77.585263) (width 0.2) (layer "F.Cu") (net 2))
 (segment (start 139.697183 77.585263) (end 139.432183 77.320263) (width 0.2) (layer "F.Cu") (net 2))
 (segment (start 135.397183 71.455263) (end 139.247183 71.455263) (width 0.2) (layer "F.Cu") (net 2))
 (segment (start 139.332183 79.450263) (end 139.347183 79.465263) (width 0.2) (layer "F.Cu") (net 2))
 (segment (start 133.717183 79.450263) (end 135.397183 79.450263) (width 0.2) (layer "F.Cu") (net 2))
 (segment (start 138.262183 77.320263) (end 138.287183 77.295263) (width 0.2) (layer "F.Cu") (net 2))
 (segment (start 133.717183 71.455263) (end 135.397183 71.455263) (width 0.2) (layer "F.Cu") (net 2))
 (segment (start 139.347183 79.465263) (end 139.697183 79.115263) (width 0.2) (layer "F.Cu") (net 2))
 (segment (start 150.462183 78.615263) (end 150.462183 77.085263) (width 0.2) (layer "F.Cu") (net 4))
 (segment (start 151.227183 75.545263) (end 151.647183 75.125263) (width 0.2) (layer "F.Cu") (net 4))
 (segment (start 150.462183 77.085263) (end 150.462183 75.545263) (width 0.2) (layer "F.Cu") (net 4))
 (segment (start 150.392183 78.295263) (end 150.362183 78.265263) (width 0.2) (layer "F.Cu") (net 4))
 (segment (start 152.977183 76.165263) (end 152.357183 75.545263) (width 0.2) (layer "F.Cu") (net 4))
 (segment (start 150.462183 75.545263) (end 151.227183 75.545263) (width 0.2) (layer "F.Cu") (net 4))
 (segment (start 150.442183 78.305263) (end 150.392183 78.355263) (width 0.2) (layer "F.Cu") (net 4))
 (segment (start 151.647183 75.125263) (end 151.647183 73.607763) (width 0.2) (layer "F.Cu") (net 4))
 (segment (start 152.357183 75.545263) (end 151.227183 75.545263) (width 0.2) (layer "F.Cu") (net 4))
 (segment (start 147.457183 73.595263) (end 147.557183 73.595263) (width 0.2) (layer "F.Cu") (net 3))
 (segment (start 145.827183 73.595263) (end 147.457183 73.595263) (width 0.2) (layer "F.Cu") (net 3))
 (segment (start 147.167183 73.650263) (end 149.062183 73.650263) (width 0.2) (layer "F.Cu") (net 3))
 (segment (start 149.287183 73.425263) (end 149.287183 72.925263) (width 0.2) (layer "F.Cu") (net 3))
 (segment (start 149.757183 72.455263) (end 151.197183 72.455263) (width 0.2) (layer "F.Cu") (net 3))
 (segment (start 151.197183 72.455263) (end 151.647183 72.005263) (width 0.2) (layer "F.Cu") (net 3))
 (segment (start 149.287183 72.925263) (end 149.757183 72.455263) (width 0.2) (layer "F.Cu") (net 3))
 (segment (start 149.062183 73.650263) (end 149.287183 73.425263) (width 0.2) (layer "F.Cu") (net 3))
 (segment (start 151.647183 72.005263) (end 151.647183 71.482763) (width 0.2) (layer "F.Cu") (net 3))
 (segment (start 143.212183 73.595263) (end 145.827183 73.595263) (width 0.2) (layer "F.Cu") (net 3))
 (segment (start 142.337183 80.525263) (end 140.777183 78.965263) (width 0.2) (layer "F.Cu") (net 5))
 (segment (start 138.262183 73.595263) (end 140.737183 73.595263) (width 0.2) (layer "F.Cu") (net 5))
 (segment (start 140.737183 73.595263) (end 141.227183 73.105263) (width 0.2) (layer "F.Cu") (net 5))
 (segment (start 141.227183 72.305263) (end 141.757183 71.775263) (width 0.2) (layer "F.Cu") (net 5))
 (segment (start 141.227183 73.105263) (end 141.227183 72.305263) (width 0.2) (layer "F.Cu") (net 5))
 (segment (start 140.777183 78.965263) (end 140.777183 73.555263) (width 0.2) (layer "F.Cu") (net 5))
 (segment (start 141.757183 71.775263) (end 142.182183 71.775263) (width 0.2) (layer "F.Cu") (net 5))
 (segment (start 140.777183 73.555263) (end 141.227183 73.105263) (width 0.2) (layer "F.Cu") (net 5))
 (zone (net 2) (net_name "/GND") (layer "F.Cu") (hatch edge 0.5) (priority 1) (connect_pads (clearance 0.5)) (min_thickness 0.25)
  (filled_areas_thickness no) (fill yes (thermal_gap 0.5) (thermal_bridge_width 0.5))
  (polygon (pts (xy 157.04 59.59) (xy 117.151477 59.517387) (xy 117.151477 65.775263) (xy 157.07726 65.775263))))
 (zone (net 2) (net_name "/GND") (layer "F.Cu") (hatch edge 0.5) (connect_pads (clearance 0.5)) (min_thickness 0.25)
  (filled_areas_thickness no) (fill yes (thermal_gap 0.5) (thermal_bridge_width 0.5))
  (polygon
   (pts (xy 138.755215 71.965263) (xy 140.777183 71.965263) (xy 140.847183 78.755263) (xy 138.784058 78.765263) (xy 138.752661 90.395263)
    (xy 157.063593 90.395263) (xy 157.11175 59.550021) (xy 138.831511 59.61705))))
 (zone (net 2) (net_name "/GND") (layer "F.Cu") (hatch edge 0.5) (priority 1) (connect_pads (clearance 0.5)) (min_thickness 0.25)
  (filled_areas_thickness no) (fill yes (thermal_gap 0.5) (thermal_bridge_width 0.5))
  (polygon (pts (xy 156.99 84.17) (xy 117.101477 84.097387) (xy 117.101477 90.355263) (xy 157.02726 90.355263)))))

